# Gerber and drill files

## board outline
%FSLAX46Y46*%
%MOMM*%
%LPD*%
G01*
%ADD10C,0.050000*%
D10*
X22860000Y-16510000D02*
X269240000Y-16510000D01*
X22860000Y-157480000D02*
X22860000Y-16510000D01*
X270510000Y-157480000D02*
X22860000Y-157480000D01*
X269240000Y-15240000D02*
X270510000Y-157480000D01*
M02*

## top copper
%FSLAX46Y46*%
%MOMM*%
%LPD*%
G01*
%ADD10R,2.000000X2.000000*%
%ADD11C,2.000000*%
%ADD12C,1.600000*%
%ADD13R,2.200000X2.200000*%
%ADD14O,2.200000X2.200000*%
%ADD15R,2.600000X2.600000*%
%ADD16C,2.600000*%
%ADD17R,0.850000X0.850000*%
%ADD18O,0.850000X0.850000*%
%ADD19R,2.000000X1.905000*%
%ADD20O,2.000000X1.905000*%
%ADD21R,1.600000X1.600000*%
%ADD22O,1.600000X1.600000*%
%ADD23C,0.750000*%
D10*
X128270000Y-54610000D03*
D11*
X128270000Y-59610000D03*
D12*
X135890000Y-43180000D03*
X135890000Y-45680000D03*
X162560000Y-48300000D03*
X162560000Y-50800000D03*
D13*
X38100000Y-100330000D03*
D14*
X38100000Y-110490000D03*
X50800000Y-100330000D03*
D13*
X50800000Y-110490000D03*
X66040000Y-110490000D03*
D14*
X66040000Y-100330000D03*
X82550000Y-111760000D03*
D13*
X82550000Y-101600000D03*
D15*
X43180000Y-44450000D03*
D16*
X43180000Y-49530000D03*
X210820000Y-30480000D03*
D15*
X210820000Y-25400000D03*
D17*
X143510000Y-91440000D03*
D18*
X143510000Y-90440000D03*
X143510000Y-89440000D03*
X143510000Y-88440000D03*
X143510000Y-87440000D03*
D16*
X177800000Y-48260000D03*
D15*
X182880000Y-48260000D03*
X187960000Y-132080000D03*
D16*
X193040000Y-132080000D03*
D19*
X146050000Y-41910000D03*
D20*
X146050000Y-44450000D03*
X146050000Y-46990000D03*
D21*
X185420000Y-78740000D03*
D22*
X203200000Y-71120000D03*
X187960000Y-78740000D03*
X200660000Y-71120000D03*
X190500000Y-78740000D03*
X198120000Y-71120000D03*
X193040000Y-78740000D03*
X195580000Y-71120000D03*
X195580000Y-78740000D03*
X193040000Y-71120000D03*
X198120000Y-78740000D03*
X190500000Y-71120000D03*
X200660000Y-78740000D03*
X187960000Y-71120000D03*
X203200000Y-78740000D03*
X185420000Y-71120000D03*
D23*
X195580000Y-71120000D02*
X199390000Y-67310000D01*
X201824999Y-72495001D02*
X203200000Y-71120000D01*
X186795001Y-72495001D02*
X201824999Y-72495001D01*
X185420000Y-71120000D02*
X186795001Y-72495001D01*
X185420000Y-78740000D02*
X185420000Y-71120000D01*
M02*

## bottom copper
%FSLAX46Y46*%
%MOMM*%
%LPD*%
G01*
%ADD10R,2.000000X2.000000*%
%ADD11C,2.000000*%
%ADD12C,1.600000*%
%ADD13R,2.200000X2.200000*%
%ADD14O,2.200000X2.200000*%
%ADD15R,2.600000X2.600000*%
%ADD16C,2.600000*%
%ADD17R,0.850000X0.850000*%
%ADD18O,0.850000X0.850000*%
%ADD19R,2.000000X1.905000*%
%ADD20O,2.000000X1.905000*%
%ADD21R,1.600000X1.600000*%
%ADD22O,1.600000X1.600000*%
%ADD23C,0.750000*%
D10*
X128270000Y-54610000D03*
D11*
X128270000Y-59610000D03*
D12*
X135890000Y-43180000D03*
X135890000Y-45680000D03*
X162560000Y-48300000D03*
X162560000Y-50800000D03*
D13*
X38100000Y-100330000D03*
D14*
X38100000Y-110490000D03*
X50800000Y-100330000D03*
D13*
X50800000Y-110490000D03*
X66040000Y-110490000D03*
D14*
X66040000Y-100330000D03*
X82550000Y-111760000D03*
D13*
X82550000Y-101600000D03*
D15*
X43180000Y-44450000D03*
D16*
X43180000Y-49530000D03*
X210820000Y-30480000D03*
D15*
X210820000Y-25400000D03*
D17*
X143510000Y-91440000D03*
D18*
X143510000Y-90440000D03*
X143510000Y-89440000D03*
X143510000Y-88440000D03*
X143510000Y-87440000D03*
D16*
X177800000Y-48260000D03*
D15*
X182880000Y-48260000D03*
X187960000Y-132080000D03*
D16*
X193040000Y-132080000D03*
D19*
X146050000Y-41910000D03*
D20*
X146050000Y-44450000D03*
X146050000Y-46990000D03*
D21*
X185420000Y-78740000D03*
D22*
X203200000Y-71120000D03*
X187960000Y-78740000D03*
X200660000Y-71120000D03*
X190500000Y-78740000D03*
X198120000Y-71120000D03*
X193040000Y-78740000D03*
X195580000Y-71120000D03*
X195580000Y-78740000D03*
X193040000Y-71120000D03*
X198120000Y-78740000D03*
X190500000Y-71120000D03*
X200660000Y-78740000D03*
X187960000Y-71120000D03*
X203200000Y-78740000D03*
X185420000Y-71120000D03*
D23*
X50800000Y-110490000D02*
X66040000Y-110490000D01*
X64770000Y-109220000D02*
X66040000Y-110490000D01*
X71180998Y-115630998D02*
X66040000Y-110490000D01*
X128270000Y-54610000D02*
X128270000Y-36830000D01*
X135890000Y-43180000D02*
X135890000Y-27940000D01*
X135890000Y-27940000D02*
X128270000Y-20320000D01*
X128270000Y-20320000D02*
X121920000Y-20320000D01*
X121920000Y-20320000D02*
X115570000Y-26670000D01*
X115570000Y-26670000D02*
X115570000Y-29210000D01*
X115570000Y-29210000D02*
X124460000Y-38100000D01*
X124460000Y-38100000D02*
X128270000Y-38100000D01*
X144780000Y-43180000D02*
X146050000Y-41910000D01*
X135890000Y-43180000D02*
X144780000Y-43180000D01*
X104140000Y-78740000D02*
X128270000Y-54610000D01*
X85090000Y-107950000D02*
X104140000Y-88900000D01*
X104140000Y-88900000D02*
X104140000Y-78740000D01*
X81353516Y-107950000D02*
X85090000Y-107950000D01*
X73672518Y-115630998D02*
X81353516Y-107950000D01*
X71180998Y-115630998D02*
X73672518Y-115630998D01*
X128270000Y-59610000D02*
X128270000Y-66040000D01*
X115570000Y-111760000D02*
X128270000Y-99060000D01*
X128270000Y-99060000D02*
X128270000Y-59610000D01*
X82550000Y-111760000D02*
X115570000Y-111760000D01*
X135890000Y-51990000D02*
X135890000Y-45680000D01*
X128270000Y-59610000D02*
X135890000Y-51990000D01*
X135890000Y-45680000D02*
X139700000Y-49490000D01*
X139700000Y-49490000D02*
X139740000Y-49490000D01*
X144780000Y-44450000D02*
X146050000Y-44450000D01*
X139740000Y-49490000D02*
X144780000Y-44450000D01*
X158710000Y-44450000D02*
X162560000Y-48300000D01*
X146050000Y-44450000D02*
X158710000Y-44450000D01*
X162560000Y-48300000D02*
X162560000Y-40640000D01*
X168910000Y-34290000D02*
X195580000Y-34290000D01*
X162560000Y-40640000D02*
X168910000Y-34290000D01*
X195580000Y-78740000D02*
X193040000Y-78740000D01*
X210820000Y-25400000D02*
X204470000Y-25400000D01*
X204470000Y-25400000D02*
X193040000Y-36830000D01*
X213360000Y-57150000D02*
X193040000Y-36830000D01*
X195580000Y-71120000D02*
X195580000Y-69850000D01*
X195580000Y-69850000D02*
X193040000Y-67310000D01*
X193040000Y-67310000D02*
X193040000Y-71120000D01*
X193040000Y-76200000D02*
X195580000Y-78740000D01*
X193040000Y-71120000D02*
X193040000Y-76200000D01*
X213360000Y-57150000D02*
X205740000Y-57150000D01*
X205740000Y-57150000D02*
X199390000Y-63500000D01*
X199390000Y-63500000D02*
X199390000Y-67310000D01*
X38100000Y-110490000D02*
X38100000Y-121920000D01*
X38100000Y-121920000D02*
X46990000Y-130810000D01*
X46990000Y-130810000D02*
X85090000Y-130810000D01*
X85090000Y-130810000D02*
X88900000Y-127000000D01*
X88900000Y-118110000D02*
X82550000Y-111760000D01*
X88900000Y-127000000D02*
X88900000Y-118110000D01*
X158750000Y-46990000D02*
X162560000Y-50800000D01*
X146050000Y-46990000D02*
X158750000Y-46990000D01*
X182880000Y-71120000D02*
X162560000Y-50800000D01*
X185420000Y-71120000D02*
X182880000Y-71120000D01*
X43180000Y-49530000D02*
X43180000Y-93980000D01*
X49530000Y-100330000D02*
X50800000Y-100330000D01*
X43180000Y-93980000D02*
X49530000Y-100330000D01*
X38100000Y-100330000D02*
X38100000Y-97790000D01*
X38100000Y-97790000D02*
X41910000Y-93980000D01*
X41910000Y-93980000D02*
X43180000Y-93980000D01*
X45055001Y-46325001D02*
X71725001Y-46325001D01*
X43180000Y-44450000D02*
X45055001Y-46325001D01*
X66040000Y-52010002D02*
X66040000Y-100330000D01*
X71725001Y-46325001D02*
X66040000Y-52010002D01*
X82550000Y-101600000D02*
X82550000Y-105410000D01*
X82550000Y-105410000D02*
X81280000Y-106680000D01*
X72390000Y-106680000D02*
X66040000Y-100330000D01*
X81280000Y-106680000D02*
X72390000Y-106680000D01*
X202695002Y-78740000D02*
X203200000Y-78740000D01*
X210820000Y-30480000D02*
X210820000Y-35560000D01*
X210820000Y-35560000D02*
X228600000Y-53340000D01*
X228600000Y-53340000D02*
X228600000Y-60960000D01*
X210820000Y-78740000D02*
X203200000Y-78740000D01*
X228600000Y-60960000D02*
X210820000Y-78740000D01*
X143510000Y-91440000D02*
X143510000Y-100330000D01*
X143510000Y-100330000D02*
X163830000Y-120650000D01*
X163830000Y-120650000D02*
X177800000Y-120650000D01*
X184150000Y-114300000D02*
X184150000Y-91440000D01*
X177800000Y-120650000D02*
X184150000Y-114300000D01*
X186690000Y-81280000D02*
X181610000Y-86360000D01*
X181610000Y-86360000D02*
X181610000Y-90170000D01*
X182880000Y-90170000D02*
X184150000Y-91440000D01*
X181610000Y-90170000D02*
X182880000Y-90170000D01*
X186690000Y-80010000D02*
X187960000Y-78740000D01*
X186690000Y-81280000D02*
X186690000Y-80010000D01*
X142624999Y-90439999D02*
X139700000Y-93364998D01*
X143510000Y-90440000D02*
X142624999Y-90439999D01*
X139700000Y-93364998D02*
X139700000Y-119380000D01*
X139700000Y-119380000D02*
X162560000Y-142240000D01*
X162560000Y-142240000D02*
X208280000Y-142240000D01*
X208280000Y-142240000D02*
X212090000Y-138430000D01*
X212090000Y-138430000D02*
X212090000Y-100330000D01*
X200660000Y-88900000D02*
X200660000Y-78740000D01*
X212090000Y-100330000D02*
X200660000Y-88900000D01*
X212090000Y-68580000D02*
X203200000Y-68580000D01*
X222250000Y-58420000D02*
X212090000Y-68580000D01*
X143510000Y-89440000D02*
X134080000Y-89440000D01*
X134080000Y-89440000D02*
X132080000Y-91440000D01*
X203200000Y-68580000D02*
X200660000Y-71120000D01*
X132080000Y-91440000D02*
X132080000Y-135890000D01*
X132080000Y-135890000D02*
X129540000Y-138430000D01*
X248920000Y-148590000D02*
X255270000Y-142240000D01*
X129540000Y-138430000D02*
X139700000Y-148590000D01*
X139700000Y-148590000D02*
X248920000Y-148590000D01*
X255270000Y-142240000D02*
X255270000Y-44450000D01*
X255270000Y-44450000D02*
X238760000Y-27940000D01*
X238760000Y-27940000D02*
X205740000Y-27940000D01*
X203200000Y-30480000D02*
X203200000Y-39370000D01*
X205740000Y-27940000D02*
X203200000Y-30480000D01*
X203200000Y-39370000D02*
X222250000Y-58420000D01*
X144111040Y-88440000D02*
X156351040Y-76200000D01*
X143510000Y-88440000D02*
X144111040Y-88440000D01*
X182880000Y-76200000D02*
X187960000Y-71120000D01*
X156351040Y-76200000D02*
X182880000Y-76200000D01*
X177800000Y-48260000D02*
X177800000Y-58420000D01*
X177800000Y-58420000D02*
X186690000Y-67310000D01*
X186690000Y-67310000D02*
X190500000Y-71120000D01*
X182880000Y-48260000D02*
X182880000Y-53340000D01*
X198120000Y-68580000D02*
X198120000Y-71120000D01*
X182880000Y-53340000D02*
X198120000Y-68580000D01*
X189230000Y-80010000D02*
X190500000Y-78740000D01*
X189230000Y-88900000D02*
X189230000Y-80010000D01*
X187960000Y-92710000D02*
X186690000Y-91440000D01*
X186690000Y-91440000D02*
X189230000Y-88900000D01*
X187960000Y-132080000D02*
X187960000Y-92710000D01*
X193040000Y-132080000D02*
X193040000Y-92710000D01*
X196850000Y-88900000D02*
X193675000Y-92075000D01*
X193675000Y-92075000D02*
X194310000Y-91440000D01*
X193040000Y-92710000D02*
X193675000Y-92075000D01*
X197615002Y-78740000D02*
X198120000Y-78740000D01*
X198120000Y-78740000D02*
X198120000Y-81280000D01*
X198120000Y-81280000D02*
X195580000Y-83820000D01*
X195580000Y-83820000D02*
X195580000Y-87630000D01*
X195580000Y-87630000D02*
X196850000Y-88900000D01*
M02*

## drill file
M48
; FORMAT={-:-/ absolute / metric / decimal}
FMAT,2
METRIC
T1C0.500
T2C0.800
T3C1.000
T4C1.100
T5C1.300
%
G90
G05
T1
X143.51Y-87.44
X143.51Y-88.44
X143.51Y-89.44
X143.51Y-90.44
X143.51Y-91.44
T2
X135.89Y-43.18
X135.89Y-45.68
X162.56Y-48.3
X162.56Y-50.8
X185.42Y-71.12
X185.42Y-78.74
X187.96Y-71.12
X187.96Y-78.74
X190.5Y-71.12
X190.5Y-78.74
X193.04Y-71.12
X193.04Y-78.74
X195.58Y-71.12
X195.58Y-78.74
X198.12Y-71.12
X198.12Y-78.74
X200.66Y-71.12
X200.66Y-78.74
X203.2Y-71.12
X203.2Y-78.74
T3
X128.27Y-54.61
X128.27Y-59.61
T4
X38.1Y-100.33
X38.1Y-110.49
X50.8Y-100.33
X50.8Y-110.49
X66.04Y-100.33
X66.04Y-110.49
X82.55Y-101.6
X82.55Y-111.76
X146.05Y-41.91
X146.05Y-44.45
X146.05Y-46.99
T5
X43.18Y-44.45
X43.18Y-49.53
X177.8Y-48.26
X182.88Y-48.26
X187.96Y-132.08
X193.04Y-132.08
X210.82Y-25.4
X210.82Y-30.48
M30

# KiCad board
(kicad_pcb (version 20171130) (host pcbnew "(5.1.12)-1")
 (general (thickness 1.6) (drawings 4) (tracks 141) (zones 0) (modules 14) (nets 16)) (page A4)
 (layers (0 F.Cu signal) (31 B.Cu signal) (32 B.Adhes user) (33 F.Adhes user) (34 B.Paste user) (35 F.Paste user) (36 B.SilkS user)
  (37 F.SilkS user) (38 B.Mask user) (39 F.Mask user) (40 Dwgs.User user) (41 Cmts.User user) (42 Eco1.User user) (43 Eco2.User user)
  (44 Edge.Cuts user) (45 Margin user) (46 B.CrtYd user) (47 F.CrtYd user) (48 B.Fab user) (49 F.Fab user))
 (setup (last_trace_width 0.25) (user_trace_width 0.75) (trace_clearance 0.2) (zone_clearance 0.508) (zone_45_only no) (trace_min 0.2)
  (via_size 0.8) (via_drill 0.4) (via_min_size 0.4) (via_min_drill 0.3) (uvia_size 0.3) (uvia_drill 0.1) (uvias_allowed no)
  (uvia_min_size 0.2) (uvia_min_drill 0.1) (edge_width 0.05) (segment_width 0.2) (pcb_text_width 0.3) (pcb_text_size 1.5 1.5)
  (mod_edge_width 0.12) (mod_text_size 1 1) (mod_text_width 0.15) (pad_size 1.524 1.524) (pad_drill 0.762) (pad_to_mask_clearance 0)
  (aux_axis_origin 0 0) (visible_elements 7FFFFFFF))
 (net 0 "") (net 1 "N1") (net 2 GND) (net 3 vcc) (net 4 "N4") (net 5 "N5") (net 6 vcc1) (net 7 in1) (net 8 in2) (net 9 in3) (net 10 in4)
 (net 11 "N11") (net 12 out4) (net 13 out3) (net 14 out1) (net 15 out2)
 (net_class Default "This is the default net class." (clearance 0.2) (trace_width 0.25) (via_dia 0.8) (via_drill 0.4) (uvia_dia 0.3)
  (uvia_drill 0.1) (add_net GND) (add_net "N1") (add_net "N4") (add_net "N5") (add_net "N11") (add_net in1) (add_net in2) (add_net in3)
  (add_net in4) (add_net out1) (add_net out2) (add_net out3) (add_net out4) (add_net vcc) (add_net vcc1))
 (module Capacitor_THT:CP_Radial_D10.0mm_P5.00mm (layer F.Cu) (at 128.27 54.61 270)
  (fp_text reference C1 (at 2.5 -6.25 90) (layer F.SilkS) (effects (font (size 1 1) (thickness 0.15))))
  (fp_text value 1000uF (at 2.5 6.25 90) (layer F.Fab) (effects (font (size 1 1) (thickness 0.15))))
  (pad 1 thru_hole rect (at 0 0 270) (size 2 2) (drill 1) (layers *.Cu *.Mask) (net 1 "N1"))
  (pad 2 thru_hole circle (at 5 0 270) (size 2 2) (drill 1) (layers *.Cu *.Mask) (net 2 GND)))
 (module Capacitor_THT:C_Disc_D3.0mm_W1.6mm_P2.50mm (layer F.Cu) (at 135.89 43.18 270)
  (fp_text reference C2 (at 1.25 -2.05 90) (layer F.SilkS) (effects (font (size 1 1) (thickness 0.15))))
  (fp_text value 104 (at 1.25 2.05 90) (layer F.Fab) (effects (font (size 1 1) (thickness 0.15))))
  (pad 1 thru_hole circle (at 0 0 270) (size 1.6 1.6) (drill 0.8) (layers *.Cu *.Mask) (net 1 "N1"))
  (pad 2 thru_hole circle (at 2.5 0 270) (size 1.6 1.6) (drill 0.8) (layers *.Cu *.Mask) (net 2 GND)))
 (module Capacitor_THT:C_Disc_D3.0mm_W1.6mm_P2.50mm (layer F.Cu) (at 162.56 50.8 90)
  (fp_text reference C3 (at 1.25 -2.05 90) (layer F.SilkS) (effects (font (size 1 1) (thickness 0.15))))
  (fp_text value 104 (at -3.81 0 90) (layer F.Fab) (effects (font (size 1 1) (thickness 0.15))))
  (pad 2 thru_hole circle (at 2.5 0 90) (size 1.6 1.6) (drill 0.8) (layers *.Cu *.Mask) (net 2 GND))
  (pad 1 thru_hole circle (at 0 0 90) (size 1.6 1.6) (drill 0.8) (layers *.Cu *.Mask) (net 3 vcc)))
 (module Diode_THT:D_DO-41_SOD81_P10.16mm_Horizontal (layer F.Cu) (at 38.1 100.33 270)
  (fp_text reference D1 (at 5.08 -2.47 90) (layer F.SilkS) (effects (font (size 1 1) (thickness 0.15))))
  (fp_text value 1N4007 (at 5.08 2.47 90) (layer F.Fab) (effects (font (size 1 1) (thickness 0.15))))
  (pad 1 thru_hole rect (at 0 0 270) (size 2.2 2.2) (drill 1.1) (layers *.Cu *.Mask) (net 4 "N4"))
  (pad 2 thru_hole oval (at 10.16 0 270) (size 2.2 2.2) (drill 1.1) (layers *.Cu *.Mask) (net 2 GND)))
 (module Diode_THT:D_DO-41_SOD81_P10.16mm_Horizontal (layer F.Cu) (at 50.8 110.49 90)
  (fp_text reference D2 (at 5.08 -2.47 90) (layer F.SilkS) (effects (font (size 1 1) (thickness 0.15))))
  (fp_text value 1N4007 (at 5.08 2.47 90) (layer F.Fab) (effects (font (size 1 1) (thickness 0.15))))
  (pad 2 thru_hole oval (at 10.16 0 90) (size 2.2 2.2) (drill 1.1) (layers *.Cu *.Mask) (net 4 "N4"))
  (pad 1 thru_hole rect (at 0 0 90) (size 2.2 2.2) (drill 1.1) (layers *.Cu *.Mask) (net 1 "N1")))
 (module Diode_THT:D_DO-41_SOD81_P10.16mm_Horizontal (layer F.Cu) (at 66.04 110.49 90)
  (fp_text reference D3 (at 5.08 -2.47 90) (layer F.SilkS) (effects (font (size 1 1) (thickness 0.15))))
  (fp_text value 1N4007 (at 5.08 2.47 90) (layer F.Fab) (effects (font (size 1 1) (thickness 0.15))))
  (pad 1 thru_hole rect (at 0 0 90) (size 2.2 2.2) (drill 1.1) (layers *.Cu *.Mask) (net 1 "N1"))
  (pad 2 thru_hole oval (at 10.16 0 90) (size 2.2 2.2) (drill 1.1) (layers *.Cu *.Mask) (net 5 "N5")))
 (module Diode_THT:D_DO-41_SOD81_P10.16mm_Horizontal (layer F.Cu) (at 82.55 101.6 270)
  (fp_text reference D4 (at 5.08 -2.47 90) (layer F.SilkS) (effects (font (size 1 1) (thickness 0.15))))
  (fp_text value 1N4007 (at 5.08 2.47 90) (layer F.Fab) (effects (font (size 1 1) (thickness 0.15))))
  (pad 2 thru_hole oval (at 10.16 0 270) (size 2.2 2.2) (drill 1.1) (layers *.Cu *.Mask) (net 2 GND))
  (pad 1 thru_hole rect (at 0 0 270) (size 2.2 2.2) (drill 1.1) (layers *.Cu *.Mask) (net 5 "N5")))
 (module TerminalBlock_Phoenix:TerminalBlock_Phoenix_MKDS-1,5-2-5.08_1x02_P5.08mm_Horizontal (layer F.Cu) (at 43.18 44.45 270)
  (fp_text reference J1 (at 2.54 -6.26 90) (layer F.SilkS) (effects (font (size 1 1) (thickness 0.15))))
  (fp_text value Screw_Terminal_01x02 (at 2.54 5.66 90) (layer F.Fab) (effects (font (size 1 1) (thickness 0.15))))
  (pad 1 thru_hole rect (at 0 0 270) (size 2.6 2.6) (drill 1.3) (layers *.Cu *.Mask) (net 5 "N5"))
  (pad 2 thru_hole circle (at 5.08 0 270) (size 2.6 2.6) (drill 1.3) (layers *.Cu *.Mask) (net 4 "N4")))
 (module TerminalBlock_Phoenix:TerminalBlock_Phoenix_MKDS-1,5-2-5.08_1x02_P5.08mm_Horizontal (layer F.Cu) (at 210.82 25.4 270)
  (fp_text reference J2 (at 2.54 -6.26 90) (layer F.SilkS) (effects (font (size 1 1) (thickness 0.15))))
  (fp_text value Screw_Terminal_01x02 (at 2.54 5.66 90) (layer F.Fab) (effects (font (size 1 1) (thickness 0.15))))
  (pad 2 thru_hole circle (at 5.08 0 270) (size 2.6 2.6) (drill 1.3) (layers *.Cu *.Mask) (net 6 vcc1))
  (pad 1 thru_hole rect (at 0 0 270) (size 2.6 2.6) (drill 1.3) (layers *.Cu *.Mask) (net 2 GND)))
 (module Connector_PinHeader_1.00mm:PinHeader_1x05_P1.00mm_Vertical (layer F.Cu) (at 143.51 91.44 180)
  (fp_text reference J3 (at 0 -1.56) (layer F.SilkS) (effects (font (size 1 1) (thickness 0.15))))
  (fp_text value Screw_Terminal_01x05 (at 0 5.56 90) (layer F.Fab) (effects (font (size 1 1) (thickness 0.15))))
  (pad 1 thru_hole rect (at 0 0 180) (size 0.85 0.85) (drill 0.5) (layers *.Cu *.Mask) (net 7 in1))
  (pad 2 thru_hole oval (at 0 1 180) (size 0.85 0.85) (drill 0.5) (layers *.Cu *.Mask) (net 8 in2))
  (pad 3 thru_hole oval (at 0 2 180) (size 0.85 0.85) (drill 0.5) (layers *.Cu *.Mask) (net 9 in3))
  (pad 4 thru_hole oval (at 0 3 180) (size 0.85 0.85) (drill 0.5) (layers *.Cu *.Mask) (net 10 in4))
  (pad 5 thru_hole oval (at 0 4 180) (size 0.85 0.85) (drill 0.5) (layers *.Cu *.Mask) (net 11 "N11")))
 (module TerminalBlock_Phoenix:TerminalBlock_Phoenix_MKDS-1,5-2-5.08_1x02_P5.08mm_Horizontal (layer F.Cu) (at 182.88 48.26 180)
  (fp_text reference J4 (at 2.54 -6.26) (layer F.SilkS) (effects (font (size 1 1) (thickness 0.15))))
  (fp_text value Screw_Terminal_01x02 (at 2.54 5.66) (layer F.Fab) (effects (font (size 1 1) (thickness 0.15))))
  (pad 2 thru_hole circle (at 5.08 0 180) (size 2.6 2.6) (drill 1.3) (layers *.Cu *.Mask) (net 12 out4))
  (pad 1 thru_hole rect (at 0 0 180) (size 2.6 2.6) (drill 1.3) (layers *.Cu *.Mask) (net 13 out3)))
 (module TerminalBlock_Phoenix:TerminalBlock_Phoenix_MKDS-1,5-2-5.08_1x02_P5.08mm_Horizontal (layer F.Cu) (at 187.96 132.08)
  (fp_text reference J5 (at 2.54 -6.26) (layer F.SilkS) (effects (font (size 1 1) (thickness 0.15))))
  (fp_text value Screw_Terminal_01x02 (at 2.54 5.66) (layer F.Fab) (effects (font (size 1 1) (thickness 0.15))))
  (pad 1 thru_hole rect (at 0 0) (size 2.6 2.6) (drill 1.3) (layers *.Cu *.Mask) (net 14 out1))
  (pad 2 thru_hole circle (at 5.08 0) (size 2.6 2.6) (drill 1.3) (layers *.Cu *.Mask) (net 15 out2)))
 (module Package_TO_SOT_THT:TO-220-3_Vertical (layer F.Cu) (at 146.05 41.91 270)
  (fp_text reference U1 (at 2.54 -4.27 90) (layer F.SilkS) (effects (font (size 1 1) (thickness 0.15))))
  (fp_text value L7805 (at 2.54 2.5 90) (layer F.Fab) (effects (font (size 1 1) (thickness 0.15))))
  (pad 1 thru_hole rect (at 0 0 270) (size 1.905 2) (drill 1.1) (layers *.Cu *.Mask) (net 1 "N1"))
  (pad 2 thru_hole oval (at 2.54 0 270) (size 1.905 2) (drill 1.1) (layers *.Cu *.Mask) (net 2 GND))
  (pad 3 thru_hole oval (at 5.08 0 270) (size 1.905 2) (drill 1.1) (layers *.Cu *.Mask) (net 3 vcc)))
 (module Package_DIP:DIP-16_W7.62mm (layer F.Cu) (at 185.42 78.74 90)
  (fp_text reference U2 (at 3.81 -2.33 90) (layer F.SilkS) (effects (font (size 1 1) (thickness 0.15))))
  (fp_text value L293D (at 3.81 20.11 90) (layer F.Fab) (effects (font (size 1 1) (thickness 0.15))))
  (pad 1 thru_hole rect (at 0 0 90) (size 1.6 1.6) (drill 0.8) (layers *.Cu *.Mask) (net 3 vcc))
  (pad 9 thru_hole oval (at 7.62 17.78 90) (size 1.6 1.6) (drill 0.8) (layers *.Cu *.Mask) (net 3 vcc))
  (pad 2 thru_hole oval (at 0 2.54 90) (size 1.6 1.6) (drill 0.8) (layers *.Cu *.Mask) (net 7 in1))
  (pad 10 thru_hole oval (at 7.62 15.24 90) (size 1.6 1.6) (drill 0.8) (layers *.Cu *.Mask) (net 9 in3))
  (pad 3 thru_hole oval (at 0 5.08 90) (size 1.6 1.6) (drill 0.8) (layers *.Cu *.Mask) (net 14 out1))
  (pad 11 thru_hole oval (at 7.62 12.7 90) (size 1.6 1.6) (drill 0.8) (layers *.Cu *.Mask) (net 13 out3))
  (pad 4 thru_hole oval (at 0 7.62 90) (size 1.6 1.6) (drill 0.8) (layers *.Cu *.Mask) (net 2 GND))
  (pad 12 thru_hole oval (at 7.62 10.16 90) (size 1.6 1.6) (drill 0.8) (layers *.Cu *.Mask) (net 2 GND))
  (pad 5 thru_hole oval (at 0 10.16 90) (size 1.6 1.6) (drill 0.8) (layers *.Cu *.Mask) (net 2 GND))
  (pad 13 thru_hole oval (at 7.62 7.62 90) (size 1.6 1.6) (drill 0.8) (layers *.Cu *.Mask) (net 2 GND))
  (pad 6 thru_hole oval (at 0 12.7 90) (size 1.6 1.6) (drill 0.8) (layers *.Cu *.Mask) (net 15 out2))
  (pad 14 thru_hole oval (at 7.62 5.08 90) (size 1.6 1.6) (drill 0.8) (layers *.Cu *.Mask) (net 12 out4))
  (pad 7 thru_hole oval (at 0 15.24 90) (size 1.6 1.6) (drill 0.8) (layers *.Cu *.Mask) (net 8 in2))
  (pad 15 thru_hole oval (at 7.62 2.54 90) (size 1.6 1.6) (drill 0.8) (layers *.Cu *.Mask) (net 10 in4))
  (pad 8 thru_hole oval (at 0 17.78 90) (size 1.6 1.6) (drill 0.8) (layers *.Cu *.Mask) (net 6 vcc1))
  (pad 16 thru_hole oval (at 7.62 0 90) (size 1.6 1.6) (drill 0.8) (layers *.Cu *.Mask) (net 3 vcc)))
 (gr_line (start 22.86 16.51) (end 269.24 16.51) (layer Edge.Cuts) (width 0.05))
 (gr_line (start 22.86 157.48) (end 22.86 16.51) (layer Edge.Cuts) (width 0.05))
 (gr_line (start 270.51 157.48) (end 22.86 157.48) (layer Edge.Cuts) (width 0.05))
 (gr_line (start 269.24 15.24) (end 270.51 157.48) (layer Edge.Cuts) (width 0.05))
 (segment (start 50.8 110.49) (end 66.04 110.49) (width 0.75) (layer B.Cu) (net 1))
 (segment (start 64.77 109.22) (end 66.04 110.49) (width 0.75) (layer B.Cu) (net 1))
 (segment (start 71.180998 115.630998) (end 66.04 110.49) (width 0.75) (layer B.Cu) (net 1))
 (segment (start 128.27 54.61) (end 128.27 36.83) (width 0.75) (layer B.Cu) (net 1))
 (segment (start 135.89 43.18) (end 135.89 27.94) (width 0.75) (layer B.Cu) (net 1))
 (segment (start 135.89 27.94) (end 128.27 20.32) (width 0.75) (layer B.Cu) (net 1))
 (segment (start 128.27 20.32) (end 121.92 20.32) (width 0.75) (layer B.Cu) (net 1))
 (segment (start 121.92 20.32) (end 115.57 26.67) (width 0.75) (layer B.Cu) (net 1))
 (segment (start 115.57 26.67) (end 115.57 29.21) (width 0.75) (layer B.Cu) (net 1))
 (segment (start 115.57 29.21) (end 124.46 38.1) (width 0.75) (layer B.Cu) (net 1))
 (segment (start 124.46 38.1) (end 128.27 38.1) (width 0.75) (layer B.Cu) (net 1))
 (segment (start 144.78 43.18) (end 146.05 41.91) (width 0.75) (layer B.Cu) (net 1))
 (segment (start 135.89 43.18) (end 144.78 43.18) (width 0.75) (layer B.Cu) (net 1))
 (segment (start 104.14 78.74) (end 128.27 54.61) (width 0.75) (layer B.Cu) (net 1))
 (segment (start 85.09 107.95) (end 104.14 88.9) (width 0.75) (layer B.Cu) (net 1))
 (segment (start 104.14 88.9) (end 104.14 78.74) (width 0.75) (layer B.Cu) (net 1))
 (segment (start 81.353516 107.95) (end 85.09 107.95) (width 0.75) (layer B.Cu) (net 1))
 (segment (start 73.672518 115.630998) (end 81.353516 107.95) (width 0.75) (layer B.Cu) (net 1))
 (segment (start 71.180998 115.630998) (end 73.672518 115.630998) (width 0.75) (layer B.Cu) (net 1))
 (segment (start 128.27 59.61) (end 128.27 66.04) (width 0.75) (layer B.Cu) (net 2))
 (segment (start 115.57 111.76) (end 128.27 99.06) (width 0.75) (layer B.Cu) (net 2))
 (segment (start 128.27 99.06) (end 128.27 59.61) (width 0.75) (layer B.Cu) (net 2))
 (segment (start 82.55 111.76) (end 115.57 111.76) (width 0.75) (layer B.Cu) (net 2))
 (segment (start 135.89 51.99) (end 135.89 45.68) (width 0.75) (layer B.Cu) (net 2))
 (segment (start 128.27 59.61) (end 135.89 51.99) (width 0.75) (layer B.Cu) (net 2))
 (segment (start 135.89 45.68) (end 139.7 49.49) (width 0.75) (layer B.Cu) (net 2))
 (segment (start 139.7 49.49) (end 139.74 49.49) (width 0.75) (layer B.Cu) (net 2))
 (segment (start 144.78 44.45) (end 146.05 44.45) (width 0.75) (layer B.Cu) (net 2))
 (segment (start 139.74 49.49) (end 144.78 44.45) (width 0.75) (layer B.Cu) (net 2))
 (segment (start 158.71 44.45) (end 162.56 48.3) (width 0.75) (layer B.Cu) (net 2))
 (segment (start 146.05 44.45) (end 158.71 44.45) (width 0.75) (layer B.Cu) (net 2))
 (segment (start 162.56 48.3) (end 162.56 40.64) (width 0.75) (layer B.Cu) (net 2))
 (segment (start 168.91 34.29) (end 195.58 34.29) (width 0.75) (layer B.Cu) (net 2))
 (segment (start 162.56 40.64) (end 168.91 34.29) (width 0.75) (layer B.Cu) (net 2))
 (segment (start 195.58 78.74) (end 193.04 78.74) (width 0.75) (layer B.Cu) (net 2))
 (segment (start 210.82 25.4) (end 204.47 25.4) (width 0.75) (layer B.Cu) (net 2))
 (segment (start 204.47 25.4) (end 193.04 36.83) (width 0.75) (layer B.Cu) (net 2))
 (segment (start 213.36 57.15) (end 193.04 36.83) (width 0.75) (layer B.Cu) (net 2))
 (segment (start 195.58 71.12) (end 195.58 69.85) (width 0.75) (layer B.Cu) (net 2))
 (segment (start 195.58 69.85) (end 193.04 67.31) (width 0.75) (layer B.Cu) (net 2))
 (segment (start 193.04 67.31) (end 193.04 71.12) (width 0.75) (layer B.Cu) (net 2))
 (segment (start 193.04 76.2) (end 195.58 78.74) (width 0.75) (layer B.Cu) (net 2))
 (segment (start 193.04 71.12) (end 193.04 76.2) (width 0.75) (layer B.Cu) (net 2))
 (segment (start 213.36 57.15) (end 205.74 57.15) (width 0.75) (layer B.Cu) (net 2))
 (segment (start 205.74 57.15) (end 199.39 63.5) (width 0.75) (layer B.Cu) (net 2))
 (segment (start 199.39 63.5) (end 199.39 67.31) (width 0.75) (layer B.Cu) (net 2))
 (segment (start 195.58 71.12) (end 199.39 67.31) (width 0.75) (layer F.Cu) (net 2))
 (segment (start 38.1 110.49) (end 38.1 121.92) (width 0.75) (layer B.Cu) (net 2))
 (segment (start 38.1 121.92) (end 46.99 130.81) (width 0.75) (layer B.Cu) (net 2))
 (segment (start 46.99 130.81) (end 85.09 130.81) (width 0.75) (layer B.Cu) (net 2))
 (segment (start 85.09 130.81) (end 88.9 127) (width 0.75) (layer B.Cu) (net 2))
 (segment (start 88.9 118.11) (end 82.55 111.76) (width 0.75) (layer B.Cu) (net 2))
 (segment (start 88.9 127) (end 88.9 118.11) (width 0.75) (layer B.Cu) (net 2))
 (segment (start 158.75 46.99) (end 162.56 50.8) (width 0.75) (layer B.Cu) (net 3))
 (segment (start 146.05 46.99) (end 158.75 46.99) (width 0.75) (layer B.Cu) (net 3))
 (segment (start 201.824999 72.495001) (end 203.2 71.12) (width 0.75) (layer F.Cu) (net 3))
 (segment (start 186.795001 72.495001) (end 201.824999 72.495001) (width 0.75) (layer F.Cu) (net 3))
 (segment (start 185.42 71.12) (end 186.795001 72.495001) (width 0.75) (layer F.Cu) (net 3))
 (segment (start 185.42 78.74) (end 185.42 71.12) (width 0.75) (layer F.Cu) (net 3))
 (segment (start 182.88 71.12) (end 162.56 50.8) (width 0.75) (layer B.Cu) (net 3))
 (segment (start 185.42 71.12) (end 182.88 71.12) (width 0.75) (layer B.Cu) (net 3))
 (segment (start 43.18 49.53) (end 43.18 93.98) (width 0.75) (layer B.Cu) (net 4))
 (segment (start 49.53 100.33) (end 50.8 100.33) (width 0.75) (layer B.Cu) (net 4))
 (segment (start 43.18 93.98) (end 49.53 100.33) (width 0.75) (layer B.Cu) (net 4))
 (segment (start 38.1 100.33) (end 38.1 97.79) (width 0.75) (layer B.Cu) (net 4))
 (segment (start 38.1 97.79) (end 41.91 93.98) (width 0.75) (layer B.Cu) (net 4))
 (segment (start 41.91 93.98) (end 43.18 93.98) (width 0.75) (layer B.Cu) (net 4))
 (segment (start 45.055001 46.325001) (end 71.725001 46.325001) (width 0.75) (layer B.Cu) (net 5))
 (segment (start 43.18 44.45) (end 45.055001 46.325001) (width 0.75) (layer B.Cu) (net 5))
 (segment (start 66.04 52.010002) (end 66.04 100.33) (width 0.75) (layer B.Cu) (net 5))
 (segment (start 71.725001 46.325001) (end 66.04 52.010002) (width 0.75) (layer B.Cu) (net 5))
 (segment (start 82.55 101.6) (end 82.55 105.41) (width 0.75) (layer B.Cu) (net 5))
 (segment (start 82.55 105.41) (end 81.28 106.68) (width 0.75) (layer B.Cu) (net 5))
 (segment (start 72.39 106.68) (end 66.04 100.33) (width 0.75) (layer B.Cu) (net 5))
 (segment (start 81.28 106.68) (end 72.39 106.68) (width 0.75) (layer B.Cu) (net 5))
 (segment (start 202.695002 78.74) (end 203.2 78.74) (width 0.75) (layer B.Cu) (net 6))
 (segment (start 210.82 30.48) (end 210.82 35.56) (width 0.75) (layer B.Cu) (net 6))
 (segment (start 210.82 35.56) (end 228.6 53.34) (width 0.75) (layer B.Cu) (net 6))
 (segment (start 228.6 53.34) (end 228.6 60.96) (width 0.75) (layer B.Cu) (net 6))
 (segment (start 210.82 78.74) (end 203.2 78.74) (width 0.75) (layer B.Cu) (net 6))
 (segment (start 228.6 60.96) (end 210.82 78.74) (width 0.75) (layer B.Cu) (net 6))
 (segment (start 143.51 91.44) (end 143.51 100.33) (width 0.75) (layer B.Cu) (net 7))
 (segment (start 143.51 100.33) (end 163.83 120.65) (width 0.75) (layer B.Cu) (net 7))
 (segment (start 163.83 120.65) (end 177.8 120.65) (width 0.75) (layer B.Cu) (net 7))
 (segment (start 184.15 114.3) (end 184.15 91.44) (width 0.75) (layer B.Cu) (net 7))
 (segment (start 177.8 120.65) (end 184.15 114.3) (width 0.75) (layer B.Cu) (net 7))
 (segment (start 186.69 81.28) (end 181.61 86.36) (width 0.75) (layer B.Cu) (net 7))
 (segment (start 181.61 86.36) (end 181.61 90.17) (width 0.75) (layer B.Cu) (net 7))
 (segment (start 182.88 90.17) (end 184.15 91.44) (width 0.75) (layer B.Cu) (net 7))
 (segment (start 181.61 90.17) (end 182.88 90.17) (width 0.75) (layer B.Cu) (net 7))
 (segment (start 186.69 80.01) (end 187.96 78.74) (width 0.75) (layer B.Cu) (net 7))
 (segment (start 186.69 81.28) (end 186.69 80.01) (width 0.75) (layer B.Cu) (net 7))
 (segment (start 142.624999 90.439999) (end 139.7 93.364998) (width 0.75) (layer B.Cu) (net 8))
 (segment (start 143.51 90.44) (end 142.624999 90.439999) (width 0.75) (layer B.Cu) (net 8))
 (segment (start 139.7 93.364998) (end 139.7 119.38) (width 0.75) (layer B.Cu) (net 8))
 (segment (start 139.7 119.38) (end 162.56 142.24) (width 0.75) (layer B.Cu) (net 8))
 (segment (start 162.56 142.24) (end 208.28 142.24) (width 0.75) (layer B.Cu) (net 8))
 (segment (start 208.28 142.24) (end 212.09 138.43) (width 0.75) (layer B.Cu) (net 8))
 (segment (start 212.09 138.43) (end 212.09 100.33) (width 0.75) (layer B.Cu) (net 8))
 (segment (start 200.66 88.9) (end 200.66 78.74) (width 0.75) (layer B.Cu) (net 8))
 (segment (start 212.09 100.33) (end 200.66 88.9) (width 0.75) (layer B.Cu) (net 8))
 (segment (start 212.09 68.58) (end 203.2 68.58) (width 0.75) (layer B.Cu) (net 9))
 (segment (start 222.25 58.42) (end 212.09 68.58) (width 0.75) (layer B.Cu) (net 9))
 (segment (start 143.51 89.44) (end 134.08 89.44) (width 0.75) (layer B.Cu) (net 9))
 (segment (start 134.08 89.44) (end 132.08 91.44) (width 0.75) (layer B.Cu) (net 9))
 (segment (start 203.2 68.58) (end 200.66 71.12) (width 0.75) (layer B.Cu) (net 9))
 (segment (start 132.08 91.44) (end 132.08 135.89) (width 0.75) (layer B.Cu) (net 9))
 (segment (start 132.08 135.89) (end 129.54 138.43) (width 0.75) (layer B.Cu) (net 9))
 (segment (start 248.92 148.59) (end 255.27 142.24) (width 0.75) (layer B.Cu) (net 9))
 (segment (start 129.54 138.43) (end 139.7 148.59) (width 0.75) (layer B.Cu) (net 9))
 (segment (start 139.7 148.59) (end 248.92 148.59) (width 0.75) (layer B.Cu) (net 9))
 (segment (start 255.27 142.24) (end 255.27 44.45) (width 0.75) (layer B.Cu) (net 9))
 (segment (start 255.27 44.45) (end 238.76 27.94) (width 0.75) (layer B.Cu) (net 9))
 (segment (start 238.76 27.94) (end 205.74 27.94) (width 0.75) (layer B.Cu) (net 9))
 (segment (start 203.2 30.48) (end 203.2 39.37) (width 0.75) (layer B.Cu) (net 9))
 (segment (start 205.74 27.94) (end 203.2 30.48) (width 0.75) (layer B.Cu) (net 9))
 (segment (start 203.2 39.37) (end 222.25 58.42) (width 0.75) (layer B.Cu) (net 9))
 (segment (start 144.11104 88.44) (end 156.35104 76.2) (width 0.75) (layer B.Cu) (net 10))
 (segment (start 143.51 88.44) (end 144.11104 88.44) (width 0.75) (layer B.Cu) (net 10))
 (segment (start 182.88 76.2) (end 187.96 71.12) (width 0.75) (layer B.Cu) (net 10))
 (segment (start 156.35104 76.2) (end 182.88 76.2) (width 0.75) (layer B.Cu) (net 10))
 (segment (start 177.8 48.26) (end 177.8 58.42) (width 0.75) (layer B.Cu) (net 12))
 (segment (start 177.8 58.42) (end 186.69 67.31) (width 0.75) (layer B.Cu) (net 12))
 (segment (start 186.69 67.31) (end 190.5 71.12) (width 0.75) (layer B.Cu) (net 12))
 (segment (start 182.88 48.26) (end 182.88 53.34) (width 0.75) (layer B.Cu) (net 13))
 (segment (start 198.12 68.58) (end 198.12 71.12) (width 0.75) (layer B.Cu) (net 13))
 (segment (start 182.88 53.34) (end 198.12 68.58) (width 0.75) (layer B.Cu) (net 13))
 (segment (start 189.23 80.01) (end 190.5 78.74) (width 0.75) (layer B.Cu) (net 14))
 (segment (start 189.23 88.9) (end 189.23 80.01) (width 0.75) (layer B.Cu) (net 14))
 (segment (start 187.96 92.71) (end 186.69 91.44) (width 0.75) (layer B.Cu) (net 14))
 (segment (start 186.69 91.44) (end 189.23 88.9) (width 0.75) (layer B.Cu) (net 14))
 (segment (start 187.96 132.08) (end 187.96 92.71) (width 0.75) (layer B.Cu) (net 14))
 (segment (start 193.04 132.08) (end 193.04 92.71) (width 0.75) (layer B.Cu) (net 15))
 (segment (start 196.85 88.9) (end 193.675 92.075) (width 0.75) (layer B.Cu) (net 15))
 (segment (start 193.675 92.075) (end 194.31 91.44) (width 0.75) (layer B.Cu) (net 15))
 (segment (start 193.04 92.71) (end 193.675 92.075) (width 0.75) (layer B.Cu) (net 15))
 (segment (start 197.615002 78.74) (end 198.12 78.74) (width 0.75) (layer B.Cu) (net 15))
 (segment (start 198.12 78.74) (end 198.12 81.28) (width 0.75) (layer B.Cu) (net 15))
 (segment (start 198.12 81.28) (end 195.58 83.82) (width 0.75) (layer B.Cu) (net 15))
 (segment (start 195.58 83.82) (end 195.58 87.63) (width 0.75) (layer B.Cu) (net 15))
 (segment (start 195.58 87.63) (end 196.85 88.9) (width 0.75) (layer B.Cu) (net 15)))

